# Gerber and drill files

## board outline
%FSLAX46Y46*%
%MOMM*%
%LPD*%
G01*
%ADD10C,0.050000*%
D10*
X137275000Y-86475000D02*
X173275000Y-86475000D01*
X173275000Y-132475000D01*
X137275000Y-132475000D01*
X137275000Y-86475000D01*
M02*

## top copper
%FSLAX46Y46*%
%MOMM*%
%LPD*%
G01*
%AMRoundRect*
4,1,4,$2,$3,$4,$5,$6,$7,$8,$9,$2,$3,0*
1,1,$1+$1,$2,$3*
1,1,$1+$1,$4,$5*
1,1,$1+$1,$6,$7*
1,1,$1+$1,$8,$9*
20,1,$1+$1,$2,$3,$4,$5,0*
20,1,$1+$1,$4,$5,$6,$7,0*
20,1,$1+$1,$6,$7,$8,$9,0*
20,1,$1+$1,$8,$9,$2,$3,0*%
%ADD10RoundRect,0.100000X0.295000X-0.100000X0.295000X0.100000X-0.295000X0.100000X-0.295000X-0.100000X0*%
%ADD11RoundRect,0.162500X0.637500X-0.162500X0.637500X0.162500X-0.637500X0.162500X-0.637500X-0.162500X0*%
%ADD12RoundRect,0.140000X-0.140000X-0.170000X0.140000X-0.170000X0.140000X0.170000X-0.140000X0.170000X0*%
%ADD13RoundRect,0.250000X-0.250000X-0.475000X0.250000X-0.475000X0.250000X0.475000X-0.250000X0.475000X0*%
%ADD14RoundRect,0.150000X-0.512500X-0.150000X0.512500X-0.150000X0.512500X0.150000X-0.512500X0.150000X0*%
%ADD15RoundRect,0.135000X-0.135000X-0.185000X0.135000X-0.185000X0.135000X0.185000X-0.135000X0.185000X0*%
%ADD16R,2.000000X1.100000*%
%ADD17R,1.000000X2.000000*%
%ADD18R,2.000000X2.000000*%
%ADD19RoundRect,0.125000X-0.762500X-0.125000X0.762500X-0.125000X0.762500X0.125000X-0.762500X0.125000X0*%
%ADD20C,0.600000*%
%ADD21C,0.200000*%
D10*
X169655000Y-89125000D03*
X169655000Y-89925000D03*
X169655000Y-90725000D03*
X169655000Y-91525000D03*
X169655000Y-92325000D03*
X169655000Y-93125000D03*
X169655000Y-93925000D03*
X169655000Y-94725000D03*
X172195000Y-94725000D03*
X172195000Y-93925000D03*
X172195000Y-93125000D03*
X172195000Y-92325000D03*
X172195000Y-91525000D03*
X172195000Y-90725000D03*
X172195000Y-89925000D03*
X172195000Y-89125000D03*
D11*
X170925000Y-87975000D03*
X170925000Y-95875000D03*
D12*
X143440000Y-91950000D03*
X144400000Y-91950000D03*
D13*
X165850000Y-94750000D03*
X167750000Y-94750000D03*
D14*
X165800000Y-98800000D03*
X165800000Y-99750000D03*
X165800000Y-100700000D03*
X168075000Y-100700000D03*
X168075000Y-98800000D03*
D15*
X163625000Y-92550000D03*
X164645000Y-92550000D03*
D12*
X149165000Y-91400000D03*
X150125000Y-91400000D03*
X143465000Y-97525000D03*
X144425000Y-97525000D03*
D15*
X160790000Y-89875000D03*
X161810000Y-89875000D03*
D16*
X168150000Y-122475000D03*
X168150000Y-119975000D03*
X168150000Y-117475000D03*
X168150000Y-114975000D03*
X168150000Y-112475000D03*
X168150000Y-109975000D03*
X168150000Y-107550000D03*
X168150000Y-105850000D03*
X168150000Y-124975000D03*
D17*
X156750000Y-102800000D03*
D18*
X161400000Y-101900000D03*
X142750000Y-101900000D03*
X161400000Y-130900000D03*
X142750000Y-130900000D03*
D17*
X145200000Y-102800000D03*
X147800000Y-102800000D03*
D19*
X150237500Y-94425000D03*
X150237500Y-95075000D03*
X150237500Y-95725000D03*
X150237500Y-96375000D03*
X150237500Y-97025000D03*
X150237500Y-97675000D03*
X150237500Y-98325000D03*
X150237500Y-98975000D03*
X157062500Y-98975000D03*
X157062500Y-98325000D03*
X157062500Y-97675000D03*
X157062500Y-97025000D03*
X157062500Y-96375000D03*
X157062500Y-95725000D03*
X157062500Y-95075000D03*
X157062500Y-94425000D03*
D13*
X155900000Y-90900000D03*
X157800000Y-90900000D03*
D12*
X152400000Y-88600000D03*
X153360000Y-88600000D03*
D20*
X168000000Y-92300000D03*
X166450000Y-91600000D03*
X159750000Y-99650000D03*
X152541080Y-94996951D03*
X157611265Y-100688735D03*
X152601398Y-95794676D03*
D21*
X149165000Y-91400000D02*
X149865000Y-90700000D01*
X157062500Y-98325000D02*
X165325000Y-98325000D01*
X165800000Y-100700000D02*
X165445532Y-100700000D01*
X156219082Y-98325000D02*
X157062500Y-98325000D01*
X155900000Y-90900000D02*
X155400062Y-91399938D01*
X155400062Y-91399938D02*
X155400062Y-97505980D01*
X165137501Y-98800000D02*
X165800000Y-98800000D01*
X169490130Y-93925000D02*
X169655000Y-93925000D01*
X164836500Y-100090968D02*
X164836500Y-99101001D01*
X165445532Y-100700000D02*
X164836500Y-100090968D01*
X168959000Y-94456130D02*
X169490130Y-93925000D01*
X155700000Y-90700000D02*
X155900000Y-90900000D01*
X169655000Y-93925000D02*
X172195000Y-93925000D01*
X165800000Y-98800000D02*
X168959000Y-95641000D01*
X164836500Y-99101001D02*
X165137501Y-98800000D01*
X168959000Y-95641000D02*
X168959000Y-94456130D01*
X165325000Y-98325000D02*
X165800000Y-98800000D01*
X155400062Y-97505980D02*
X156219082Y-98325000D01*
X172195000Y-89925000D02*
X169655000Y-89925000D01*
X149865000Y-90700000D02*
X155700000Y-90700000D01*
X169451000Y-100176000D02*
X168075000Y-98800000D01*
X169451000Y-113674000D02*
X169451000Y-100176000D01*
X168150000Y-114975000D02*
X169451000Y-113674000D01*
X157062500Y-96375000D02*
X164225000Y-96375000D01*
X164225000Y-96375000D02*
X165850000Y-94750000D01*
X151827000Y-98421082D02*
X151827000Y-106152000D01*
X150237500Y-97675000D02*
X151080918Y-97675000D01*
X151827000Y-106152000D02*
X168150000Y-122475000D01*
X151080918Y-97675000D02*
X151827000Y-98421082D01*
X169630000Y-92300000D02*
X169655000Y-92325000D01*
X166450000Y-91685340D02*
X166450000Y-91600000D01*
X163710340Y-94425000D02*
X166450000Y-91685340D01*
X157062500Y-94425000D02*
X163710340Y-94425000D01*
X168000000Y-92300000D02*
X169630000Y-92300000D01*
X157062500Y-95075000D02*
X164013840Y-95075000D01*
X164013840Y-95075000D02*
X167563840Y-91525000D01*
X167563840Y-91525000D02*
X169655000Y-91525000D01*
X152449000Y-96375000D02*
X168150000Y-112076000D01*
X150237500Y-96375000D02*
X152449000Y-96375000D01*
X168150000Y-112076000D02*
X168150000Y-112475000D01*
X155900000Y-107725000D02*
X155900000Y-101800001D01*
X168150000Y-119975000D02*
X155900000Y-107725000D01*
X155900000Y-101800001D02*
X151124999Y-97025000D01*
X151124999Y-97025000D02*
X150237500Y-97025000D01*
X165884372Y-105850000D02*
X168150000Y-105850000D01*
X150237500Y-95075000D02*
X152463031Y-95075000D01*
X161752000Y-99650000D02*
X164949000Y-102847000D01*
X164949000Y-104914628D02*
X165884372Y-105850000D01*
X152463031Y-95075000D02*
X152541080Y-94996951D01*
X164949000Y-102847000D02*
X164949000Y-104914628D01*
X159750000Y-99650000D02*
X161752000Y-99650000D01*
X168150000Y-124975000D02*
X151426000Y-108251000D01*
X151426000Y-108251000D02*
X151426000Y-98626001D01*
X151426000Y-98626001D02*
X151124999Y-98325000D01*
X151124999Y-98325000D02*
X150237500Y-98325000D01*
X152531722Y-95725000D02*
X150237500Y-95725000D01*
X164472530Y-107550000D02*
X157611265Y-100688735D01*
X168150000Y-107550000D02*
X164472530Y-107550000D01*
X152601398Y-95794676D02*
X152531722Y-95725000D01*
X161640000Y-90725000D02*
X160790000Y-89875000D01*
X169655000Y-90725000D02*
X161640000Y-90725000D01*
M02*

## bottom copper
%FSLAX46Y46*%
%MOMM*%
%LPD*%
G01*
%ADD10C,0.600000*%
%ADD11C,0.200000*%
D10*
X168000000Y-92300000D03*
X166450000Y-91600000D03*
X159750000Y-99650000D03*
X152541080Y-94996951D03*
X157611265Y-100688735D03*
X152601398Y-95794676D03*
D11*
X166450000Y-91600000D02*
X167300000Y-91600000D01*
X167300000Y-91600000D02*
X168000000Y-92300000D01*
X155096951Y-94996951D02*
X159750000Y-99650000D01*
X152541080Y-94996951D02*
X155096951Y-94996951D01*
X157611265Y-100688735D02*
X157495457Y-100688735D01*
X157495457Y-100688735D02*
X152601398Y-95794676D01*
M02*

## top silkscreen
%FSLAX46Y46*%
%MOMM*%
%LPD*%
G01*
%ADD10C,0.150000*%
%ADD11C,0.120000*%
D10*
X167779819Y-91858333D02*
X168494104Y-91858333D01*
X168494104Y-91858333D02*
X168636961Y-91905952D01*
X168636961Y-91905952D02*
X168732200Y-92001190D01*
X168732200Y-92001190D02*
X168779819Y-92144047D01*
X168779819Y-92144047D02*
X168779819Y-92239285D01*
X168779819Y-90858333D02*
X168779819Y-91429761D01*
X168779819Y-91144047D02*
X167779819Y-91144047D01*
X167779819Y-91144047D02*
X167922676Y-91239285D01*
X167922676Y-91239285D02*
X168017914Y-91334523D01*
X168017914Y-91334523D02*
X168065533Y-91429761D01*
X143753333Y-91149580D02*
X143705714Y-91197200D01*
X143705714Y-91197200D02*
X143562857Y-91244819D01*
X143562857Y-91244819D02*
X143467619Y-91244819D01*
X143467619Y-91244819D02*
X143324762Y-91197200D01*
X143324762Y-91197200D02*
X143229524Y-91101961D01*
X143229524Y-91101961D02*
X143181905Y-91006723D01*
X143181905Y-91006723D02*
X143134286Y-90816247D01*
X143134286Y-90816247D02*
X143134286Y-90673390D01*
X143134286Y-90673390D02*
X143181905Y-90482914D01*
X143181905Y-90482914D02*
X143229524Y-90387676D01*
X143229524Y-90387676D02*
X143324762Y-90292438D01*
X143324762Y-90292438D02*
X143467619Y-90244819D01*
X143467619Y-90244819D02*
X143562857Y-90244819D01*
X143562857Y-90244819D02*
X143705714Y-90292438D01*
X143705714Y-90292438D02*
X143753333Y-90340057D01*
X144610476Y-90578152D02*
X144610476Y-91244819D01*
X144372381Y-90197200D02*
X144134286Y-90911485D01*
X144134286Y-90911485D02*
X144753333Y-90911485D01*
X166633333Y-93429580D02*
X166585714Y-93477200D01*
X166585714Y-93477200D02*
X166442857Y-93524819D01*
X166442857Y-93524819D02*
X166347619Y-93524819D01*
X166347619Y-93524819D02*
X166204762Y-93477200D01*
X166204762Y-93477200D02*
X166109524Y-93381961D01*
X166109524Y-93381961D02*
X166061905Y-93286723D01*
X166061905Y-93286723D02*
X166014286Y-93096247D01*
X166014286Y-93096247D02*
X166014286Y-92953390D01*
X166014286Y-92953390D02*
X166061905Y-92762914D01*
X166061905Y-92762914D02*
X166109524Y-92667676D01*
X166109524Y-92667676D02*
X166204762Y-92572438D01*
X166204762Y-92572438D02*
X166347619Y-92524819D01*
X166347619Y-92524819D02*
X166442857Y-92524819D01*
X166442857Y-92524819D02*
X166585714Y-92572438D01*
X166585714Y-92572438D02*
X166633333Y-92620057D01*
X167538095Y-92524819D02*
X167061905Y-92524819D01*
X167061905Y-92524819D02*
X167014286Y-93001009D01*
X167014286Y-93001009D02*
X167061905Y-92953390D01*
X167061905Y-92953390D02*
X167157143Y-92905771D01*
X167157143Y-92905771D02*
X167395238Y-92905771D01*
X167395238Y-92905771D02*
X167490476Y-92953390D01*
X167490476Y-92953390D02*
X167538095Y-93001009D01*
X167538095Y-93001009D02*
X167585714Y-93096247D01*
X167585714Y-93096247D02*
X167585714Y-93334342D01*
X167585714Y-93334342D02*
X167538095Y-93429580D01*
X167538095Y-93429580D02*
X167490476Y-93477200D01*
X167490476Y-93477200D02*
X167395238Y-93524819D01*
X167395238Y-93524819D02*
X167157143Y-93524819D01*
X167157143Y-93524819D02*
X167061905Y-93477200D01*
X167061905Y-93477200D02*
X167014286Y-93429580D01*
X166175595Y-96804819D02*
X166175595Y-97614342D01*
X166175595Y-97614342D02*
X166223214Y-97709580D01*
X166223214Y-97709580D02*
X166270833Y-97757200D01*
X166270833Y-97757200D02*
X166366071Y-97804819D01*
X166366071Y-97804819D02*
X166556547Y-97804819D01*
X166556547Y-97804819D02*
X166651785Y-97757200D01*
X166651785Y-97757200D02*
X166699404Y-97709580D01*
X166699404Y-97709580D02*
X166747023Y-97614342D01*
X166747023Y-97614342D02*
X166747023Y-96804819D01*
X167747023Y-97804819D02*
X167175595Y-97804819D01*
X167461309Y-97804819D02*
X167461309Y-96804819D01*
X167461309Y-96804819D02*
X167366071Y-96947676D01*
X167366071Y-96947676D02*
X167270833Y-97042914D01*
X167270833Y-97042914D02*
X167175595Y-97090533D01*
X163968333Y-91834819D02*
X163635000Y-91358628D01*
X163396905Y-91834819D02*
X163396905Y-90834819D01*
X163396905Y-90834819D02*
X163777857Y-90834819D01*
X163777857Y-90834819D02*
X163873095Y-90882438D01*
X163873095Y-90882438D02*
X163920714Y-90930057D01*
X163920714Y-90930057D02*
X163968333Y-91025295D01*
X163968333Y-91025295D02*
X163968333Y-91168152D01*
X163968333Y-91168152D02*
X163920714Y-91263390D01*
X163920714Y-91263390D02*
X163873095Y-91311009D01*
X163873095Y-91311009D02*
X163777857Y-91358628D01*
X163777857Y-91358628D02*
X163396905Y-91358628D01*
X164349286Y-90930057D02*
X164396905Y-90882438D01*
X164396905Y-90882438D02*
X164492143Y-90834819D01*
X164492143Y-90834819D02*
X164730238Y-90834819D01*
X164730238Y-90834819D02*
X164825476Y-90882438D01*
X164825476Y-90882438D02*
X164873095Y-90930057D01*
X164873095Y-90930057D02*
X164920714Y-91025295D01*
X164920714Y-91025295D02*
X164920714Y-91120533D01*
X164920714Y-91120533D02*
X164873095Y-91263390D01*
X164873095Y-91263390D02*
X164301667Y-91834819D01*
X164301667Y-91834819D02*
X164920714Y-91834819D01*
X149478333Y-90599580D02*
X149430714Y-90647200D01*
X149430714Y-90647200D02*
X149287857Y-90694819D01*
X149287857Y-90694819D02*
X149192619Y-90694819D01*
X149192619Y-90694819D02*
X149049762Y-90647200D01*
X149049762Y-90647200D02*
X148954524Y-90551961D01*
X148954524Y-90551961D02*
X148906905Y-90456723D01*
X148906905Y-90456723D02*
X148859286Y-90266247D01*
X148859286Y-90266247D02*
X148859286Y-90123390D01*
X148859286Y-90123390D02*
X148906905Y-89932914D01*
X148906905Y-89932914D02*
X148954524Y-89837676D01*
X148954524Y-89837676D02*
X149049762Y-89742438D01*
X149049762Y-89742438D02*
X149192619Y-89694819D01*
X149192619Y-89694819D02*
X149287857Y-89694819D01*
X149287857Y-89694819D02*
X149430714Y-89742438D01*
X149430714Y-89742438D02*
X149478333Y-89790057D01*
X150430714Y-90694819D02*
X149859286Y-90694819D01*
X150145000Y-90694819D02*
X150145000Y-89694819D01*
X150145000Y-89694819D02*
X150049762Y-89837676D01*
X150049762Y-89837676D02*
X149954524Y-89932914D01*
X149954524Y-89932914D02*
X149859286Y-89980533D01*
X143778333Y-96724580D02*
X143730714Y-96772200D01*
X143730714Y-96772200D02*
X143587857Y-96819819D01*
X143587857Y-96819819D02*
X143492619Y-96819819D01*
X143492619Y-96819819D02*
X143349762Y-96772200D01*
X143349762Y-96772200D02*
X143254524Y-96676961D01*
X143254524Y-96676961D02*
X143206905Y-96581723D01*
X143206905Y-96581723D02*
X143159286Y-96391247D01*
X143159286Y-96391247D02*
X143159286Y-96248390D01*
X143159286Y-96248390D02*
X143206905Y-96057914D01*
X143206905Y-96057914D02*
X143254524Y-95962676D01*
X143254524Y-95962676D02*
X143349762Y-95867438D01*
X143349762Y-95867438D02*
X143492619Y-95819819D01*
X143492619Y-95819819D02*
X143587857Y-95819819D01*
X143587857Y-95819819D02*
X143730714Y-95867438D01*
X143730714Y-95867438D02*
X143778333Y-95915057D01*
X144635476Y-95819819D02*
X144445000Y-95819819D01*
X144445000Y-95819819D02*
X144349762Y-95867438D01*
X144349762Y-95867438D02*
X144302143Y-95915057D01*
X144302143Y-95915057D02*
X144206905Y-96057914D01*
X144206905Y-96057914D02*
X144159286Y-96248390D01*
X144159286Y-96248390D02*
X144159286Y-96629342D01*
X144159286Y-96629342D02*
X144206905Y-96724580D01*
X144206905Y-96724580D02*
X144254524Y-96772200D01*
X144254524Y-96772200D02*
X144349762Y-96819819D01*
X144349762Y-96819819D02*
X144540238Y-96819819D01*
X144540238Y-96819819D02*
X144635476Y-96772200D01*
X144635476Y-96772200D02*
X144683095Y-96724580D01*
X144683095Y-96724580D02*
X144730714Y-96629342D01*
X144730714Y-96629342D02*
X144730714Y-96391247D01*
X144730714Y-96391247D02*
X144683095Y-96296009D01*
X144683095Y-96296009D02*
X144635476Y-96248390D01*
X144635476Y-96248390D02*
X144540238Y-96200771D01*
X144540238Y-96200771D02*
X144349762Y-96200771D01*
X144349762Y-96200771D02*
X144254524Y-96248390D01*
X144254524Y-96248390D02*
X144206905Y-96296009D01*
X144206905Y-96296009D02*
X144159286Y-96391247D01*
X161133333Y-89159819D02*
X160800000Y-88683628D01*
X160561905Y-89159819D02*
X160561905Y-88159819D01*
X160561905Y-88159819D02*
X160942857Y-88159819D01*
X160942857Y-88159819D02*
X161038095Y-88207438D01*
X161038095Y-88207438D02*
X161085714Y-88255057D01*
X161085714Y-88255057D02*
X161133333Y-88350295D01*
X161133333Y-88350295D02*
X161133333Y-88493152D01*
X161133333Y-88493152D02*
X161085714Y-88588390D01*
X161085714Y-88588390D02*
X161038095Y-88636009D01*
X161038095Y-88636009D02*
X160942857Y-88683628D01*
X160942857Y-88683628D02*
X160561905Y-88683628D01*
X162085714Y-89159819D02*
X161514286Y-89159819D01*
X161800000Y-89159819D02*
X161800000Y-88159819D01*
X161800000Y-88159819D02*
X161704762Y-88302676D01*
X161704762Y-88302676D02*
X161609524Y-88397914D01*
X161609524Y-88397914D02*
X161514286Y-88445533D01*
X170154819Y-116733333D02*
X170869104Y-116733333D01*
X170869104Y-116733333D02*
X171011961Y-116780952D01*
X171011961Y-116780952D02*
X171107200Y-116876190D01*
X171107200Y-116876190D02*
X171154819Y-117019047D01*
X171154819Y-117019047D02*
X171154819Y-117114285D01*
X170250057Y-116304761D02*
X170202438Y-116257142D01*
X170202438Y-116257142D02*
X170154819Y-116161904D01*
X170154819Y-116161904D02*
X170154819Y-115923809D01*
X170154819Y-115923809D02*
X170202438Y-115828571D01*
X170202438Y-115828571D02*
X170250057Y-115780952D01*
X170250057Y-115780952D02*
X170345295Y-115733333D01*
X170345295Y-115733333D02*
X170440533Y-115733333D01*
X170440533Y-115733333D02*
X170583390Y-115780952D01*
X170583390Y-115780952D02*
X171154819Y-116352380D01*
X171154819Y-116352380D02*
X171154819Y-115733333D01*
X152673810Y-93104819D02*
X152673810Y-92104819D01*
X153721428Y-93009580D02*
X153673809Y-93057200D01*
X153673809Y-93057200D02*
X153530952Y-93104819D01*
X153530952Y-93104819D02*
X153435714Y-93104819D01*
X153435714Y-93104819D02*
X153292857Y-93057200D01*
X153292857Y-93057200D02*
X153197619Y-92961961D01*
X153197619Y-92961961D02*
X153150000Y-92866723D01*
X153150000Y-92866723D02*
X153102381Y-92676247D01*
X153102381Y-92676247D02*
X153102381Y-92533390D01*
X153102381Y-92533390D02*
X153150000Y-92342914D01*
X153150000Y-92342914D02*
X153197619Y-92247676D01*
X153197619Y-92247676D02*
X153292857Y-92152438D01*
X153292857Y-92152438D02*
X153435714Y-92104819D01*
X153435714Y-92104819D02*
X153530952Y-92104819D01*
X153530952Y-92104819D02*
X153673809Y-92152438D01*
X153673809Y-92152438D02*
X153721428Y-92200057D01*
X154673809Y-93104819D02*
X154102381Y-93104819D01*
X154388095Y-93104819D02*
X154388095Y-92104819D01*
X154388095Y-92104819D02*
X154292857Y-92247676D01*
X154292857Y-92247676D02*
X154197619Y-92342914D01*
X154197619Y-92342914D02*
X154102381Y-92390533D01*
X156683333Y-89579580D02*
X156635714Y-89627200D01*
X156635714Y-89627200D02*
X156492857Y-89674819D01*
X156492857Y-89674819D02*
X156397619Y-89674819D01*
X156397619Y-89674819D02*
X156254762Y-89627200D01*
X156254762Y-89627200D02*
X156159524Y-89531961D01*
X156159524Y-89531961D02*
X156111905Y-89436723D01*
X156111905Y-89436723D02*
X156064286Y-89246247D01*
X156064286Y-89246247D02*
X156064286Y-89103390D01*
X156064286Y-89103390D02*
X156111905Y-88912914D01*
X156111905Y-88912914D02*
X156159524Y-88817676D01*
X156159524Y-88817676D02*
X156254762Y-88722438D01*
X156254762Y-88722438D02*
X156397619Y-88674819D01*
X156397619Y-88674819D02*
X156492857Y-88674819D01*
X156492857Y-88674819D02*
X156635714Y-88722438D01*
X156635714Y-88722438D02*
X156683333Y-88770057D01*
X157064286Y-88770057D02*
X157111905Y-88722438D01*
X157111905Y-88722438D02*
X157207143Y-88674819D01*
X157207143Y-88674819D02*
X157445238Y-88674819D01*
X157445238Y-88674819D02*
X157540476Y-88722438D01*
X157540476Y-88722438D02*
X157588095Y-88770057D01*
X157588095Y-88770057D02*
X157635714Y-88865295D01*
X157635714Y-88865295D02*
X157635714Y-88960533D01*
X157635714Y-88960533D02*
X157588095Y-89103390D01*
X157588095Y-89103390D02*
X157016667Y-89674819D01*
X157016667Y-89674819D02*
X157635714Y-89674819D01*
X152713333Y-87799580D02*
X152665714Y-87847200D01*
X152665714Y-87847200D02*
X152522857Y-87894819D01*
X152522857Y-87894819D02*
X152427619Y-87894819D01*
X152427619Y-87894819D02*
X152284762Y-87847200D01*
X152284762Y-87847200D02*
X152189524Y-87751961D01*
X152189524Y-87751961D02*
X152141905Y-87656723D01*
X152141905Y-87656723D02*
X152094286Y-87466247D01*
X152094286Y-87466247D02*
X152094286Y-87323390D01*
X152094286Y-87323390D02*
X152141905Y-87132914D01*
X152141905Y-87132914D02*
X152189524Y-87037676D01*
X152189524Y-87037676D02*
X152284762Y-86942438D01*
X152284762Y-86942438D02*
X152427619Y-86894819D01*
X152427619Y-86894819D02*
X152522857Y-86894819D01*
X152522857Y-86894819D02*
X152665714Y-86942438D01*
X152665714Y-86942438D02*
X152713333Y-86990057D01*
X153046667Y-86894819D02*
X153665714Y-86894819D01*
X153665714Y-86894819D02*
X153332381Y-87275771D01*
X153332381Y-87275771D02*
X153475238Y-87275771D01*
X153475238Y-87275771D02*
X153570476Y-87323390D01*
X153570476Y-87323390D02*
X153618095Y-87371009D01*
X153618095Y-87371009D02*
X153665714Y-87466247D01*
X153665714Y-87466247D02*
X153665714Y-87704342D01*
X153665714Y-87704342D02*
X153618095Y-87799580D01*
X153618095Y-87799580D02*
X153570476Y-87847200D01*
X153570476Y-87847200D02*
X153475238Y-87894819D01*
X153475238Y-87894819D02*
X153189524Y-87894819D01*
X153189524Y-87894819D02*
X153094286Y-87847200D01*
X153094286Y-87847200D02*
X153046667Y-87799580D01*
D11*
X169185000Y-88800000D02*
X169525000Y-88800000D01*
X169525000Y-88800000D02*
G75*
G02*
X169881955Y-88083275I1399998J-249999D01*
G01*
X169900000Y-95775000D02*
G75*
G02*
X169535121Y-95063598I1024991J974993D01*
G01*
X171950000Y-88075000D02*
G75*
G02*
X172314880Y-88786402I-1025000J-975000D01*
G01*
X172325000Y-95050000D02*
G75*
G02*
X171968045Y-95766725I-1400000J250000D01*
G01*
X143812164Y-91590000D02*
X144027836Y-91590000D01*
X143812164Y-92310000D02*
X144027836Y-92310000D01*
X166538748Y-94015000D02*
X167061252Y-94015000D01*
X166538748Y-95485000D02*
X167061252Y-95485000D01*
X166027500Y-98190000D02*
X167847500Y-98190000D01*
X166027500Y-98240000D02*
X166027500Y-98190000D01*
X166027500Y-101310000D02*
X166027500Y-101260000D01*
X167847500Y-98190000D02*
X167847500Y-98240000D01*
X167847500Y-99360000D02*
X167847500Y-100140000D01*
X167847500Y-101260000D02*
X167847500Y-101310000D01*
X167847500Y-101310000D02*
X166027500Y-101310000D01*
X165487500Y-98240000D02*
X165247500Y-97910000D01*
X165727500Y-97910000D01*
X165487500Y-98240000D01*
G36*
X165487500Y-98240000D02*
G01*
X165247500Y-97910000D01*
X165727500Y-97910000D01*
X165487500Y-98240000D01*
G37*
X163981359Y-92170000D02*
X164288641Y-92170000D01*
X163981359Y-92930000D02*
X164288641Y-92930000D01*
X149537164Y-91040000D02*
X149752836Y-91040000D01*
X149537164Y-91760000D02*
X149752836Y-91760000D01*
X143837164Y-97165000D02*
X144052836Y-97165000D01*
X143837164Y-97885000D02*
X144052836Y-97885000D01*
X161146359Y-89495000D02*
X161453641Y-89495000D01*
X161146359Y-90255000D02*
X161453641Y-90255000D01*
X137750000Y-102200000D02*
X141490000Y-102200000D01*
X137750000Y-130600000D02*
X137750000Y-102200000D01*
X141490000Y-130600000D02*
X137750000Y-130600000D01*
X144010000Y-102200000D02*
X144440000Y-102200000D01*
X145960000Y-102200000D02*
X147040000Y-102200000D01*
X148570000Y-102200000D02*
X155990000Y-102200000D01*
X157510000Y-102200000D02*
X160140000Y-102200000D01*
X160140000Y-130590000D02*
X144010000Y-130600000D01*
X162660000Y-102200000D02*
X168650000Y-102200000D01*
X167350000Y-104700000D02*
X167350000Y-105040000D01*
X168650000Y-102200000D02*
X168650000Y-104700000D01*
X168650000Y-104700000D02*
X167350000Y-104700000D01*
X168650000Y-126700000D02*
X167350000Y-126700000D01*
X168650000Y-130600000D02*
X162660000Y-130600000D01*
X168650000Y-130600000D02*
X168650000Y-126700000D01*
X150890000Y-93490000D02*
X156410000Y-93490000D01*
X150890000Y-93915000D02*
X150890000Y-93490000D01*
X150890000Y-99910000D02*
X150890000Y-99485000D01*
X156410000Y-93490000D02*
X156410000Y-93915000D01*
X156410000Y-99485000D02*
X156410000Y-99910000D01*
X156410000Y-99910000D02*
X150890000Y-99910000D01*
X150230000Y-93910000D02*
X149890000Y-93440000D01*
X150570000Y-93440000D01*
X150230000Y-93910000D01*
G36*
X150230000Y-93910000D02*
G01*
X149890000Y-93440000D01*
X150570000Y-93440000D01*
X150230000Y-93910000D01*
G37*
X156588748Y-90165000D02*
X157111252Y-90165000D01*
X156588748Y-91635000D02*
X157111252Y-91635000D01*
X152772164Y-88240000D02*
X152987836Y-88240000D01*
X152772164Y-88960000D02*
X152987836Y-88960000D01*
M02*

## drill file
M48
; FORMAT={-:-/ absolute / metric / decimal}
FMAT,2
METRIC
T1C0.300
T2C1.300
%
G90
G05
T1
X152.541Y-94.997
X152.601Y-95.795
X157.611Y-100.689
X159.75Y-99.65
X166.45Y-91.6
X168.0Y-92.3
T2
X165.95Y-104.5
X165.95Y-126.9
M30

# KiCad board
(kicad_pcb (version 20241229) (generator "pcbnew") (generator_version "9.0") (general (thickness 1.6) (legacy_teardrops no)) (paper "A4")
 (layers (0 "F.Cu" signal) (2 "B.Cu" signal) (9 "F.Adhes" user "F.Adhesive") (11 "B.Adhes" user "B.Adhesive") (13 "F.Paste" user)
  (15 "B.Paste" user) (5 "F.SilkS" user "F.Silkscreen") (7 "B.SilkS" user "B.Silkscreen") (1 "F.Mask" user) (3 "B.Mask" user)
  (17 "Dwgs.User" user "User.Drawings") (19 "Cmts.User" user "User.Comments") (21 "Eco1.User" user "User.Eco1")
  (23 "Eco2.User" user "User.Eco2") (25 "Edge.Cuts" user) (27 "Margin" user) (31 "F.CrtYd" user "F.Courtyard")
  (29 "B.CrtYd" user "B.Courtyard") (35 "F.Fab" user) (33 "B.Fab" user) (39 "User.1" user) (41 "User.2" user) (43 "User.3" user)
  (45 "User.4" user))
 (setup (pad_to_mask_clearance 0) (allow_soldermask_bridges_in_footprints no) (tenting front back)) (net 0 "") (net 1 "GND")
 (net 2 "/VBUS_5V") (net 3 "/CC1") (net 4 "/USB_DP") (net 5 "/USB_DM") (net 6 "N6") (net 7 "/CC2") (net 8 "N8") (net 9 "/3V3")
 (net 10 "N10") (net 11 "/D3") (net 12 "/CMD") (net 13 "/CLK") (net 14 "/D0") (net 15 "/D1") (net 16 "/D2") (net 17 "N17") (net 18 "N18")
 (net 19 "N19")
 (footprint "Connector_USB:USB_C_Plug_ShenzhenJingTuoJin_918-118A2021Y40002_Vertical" (layer "F.Cu") (at 170.925 91.925)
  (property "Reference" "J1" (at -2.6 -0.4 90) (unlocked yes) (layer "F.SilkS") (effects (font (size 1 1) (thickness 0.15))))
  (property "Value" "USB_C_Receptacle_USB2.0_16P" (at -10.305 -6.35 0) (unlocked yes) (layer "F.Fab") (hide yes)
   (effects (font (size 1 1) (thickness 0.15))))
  (fp_line (start -1.74 -3.125) (end -1.4 -3.125) (stroke (width 0.12) (type default)) (layer "F.SilkS"))
  (fp_arc (start -1.4 -3.125) (mid -1.273005 -3.509002) (end -1.043045 -3.841725) (stroke (width 0.12) (type solid)) (layer "F.SilkS"))
  (fp_arc (start -1.025 3.85) (mid -1.258743 3.520613) (end -1.389879 3.138598) (stroke (width 0.12) (type solid)) (layer "F.SilkS"))
  (fp_arc (start 1.025 -3.85) (mid 1.258743 -3.520613) (end 1.389879 -3.138598) (stroke (width 0.12) (type solid)) (layer "F.SilkS"))
  (fp_arc (start 1.4 3.125) (mid 1.273005 3.509002) (end 1.043045 3.841725) (stroke (width 0.12) (type solid)) (layer "F.SilkS"))
  (pad "A1" smd roundrect (at -1.27 -2.8 90) (size 0.4 0.79) (layers "F.Cu" "F.Mask" "F.Paste") (roundrect_rratio 0.25) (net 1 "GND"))
  (pad "A4" smd roundrect (at -1.27 -2 90) (size 0.4 0.79) (layers "F.Cu" "F.Mask" "F.Paste") (roundrect_rratio 0.25) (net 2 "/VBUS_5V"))
  (pad "A5" smd roundrect (at -1.27 -1.2 90) (size 0.4 0.79) (layers "F.Cu" "F.Mask" "F.Paste") (roundrect_rratio 0.25) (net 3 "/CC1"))
  (pad "A6" smd roundrect (at -1.27 -0.4 90) (size 0.4 0.79) (layers "F.Cu" "F.Mask" "F.Paste") (roundrect_rratio 0.25) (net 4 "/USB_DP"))
  (pad "A7" smd roundrect (at -1.27 0.4 90) (size 0.4 0.79) (layers "F.Cu" "F.Mask" "F.Paste") (roundrect_rratio 0.25) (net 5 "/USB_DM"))
  (pad "A8" smd roundrect (at -1.27 1.2 90) (size 0.4 0.79) (layers "F.Cu" "F.Mask" "F.Paste") (roundrect_rratio 0.25) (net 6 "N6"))
  (pad "A9" smd roundrect (at -1.27 2 90) (size 0.4 0.79) (layers "F.Cu" "F.Mask" "F.Paste") (roundrect_rratio 0.25) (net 2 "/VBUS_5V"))
  (pad "A12" smd roundrect (at -1.27 2.8 90) (size 0.4 0.79) (layers "F.Cu" "F.Mask" "F.Paste") (roundrect_rratio 0.25) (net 1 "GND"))
  (pad "B1" smd roundrect (at 1.27 2.8 90) (size 0.4 0.79) (layers "F.Cu" "F.Mask" "F.Paste") (roundrect_rratio 0.25) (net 1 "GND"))
  (pad "B4" smd roundrect (at 1.27 2 90) (size 0.4 0.79) (layers "F.Cu" "F.Mask" "F.Paste") (roundrect_rratio 0.25) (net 2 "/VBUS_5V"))
  (pad "B5" smd roundrect (at 1.27 1.2 90) (size 0.4 0.79) (layers "F.Cu" "F.Mask" "F.Paste") (roundrect_rratio 0.25) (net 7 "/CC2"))
  (pad "B6" smd roundrect (at 1.27 0.4 90) (size 0.4 0.79) (layers "F.Cu" "F.Mask" "F.Paste") (roundrect_rratio 0.25) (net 4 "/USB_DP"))
  (pad "B7" smd roundrect (at 1.27 -0.4 90) (size 0.4 0.79) (layers "F.Cu" "F.Mask" "F.Paste") (roundrect_rratio 0.25) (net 5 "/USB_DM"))
  (pad "B8" smd roundrect (at 1.27 -1.2 90) (size 0.4 0.79) (layers "F.Cu" "F.Mask" "F.Paste") (roundrect_rratio 0.25) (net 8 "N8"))
  (pad "B9" smd roundrect (at 1.27 -2 90) (size 0.4 0.79) (layers "F.Cu" "F.Mask" "F.Paste") (roundrect_rratio 0.25) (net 2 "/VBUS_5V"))
  (pad "B12" smd roundrect (at 1.27 -2.8 90) (size 0.4 0.79) (layers "F.Cu" "F.Mask" "F.Paste") (roundrect_rratio 0.25) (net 1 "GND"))
  (pad "S1" smd roundrect (at 0 -3.95 90) (size 0.65 1.6) (layers "F.Cu" "F.Mask" "F.Paste") (roundrect_rratio 0.25) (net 1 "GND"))
  (pad "S1" smd roundrect (at 0 3.95 90) (size 0.65 1.6) (layers "F.Cu" "F.Mask" "F.Paste") (roundrect_rratio 0.25) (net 1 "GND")))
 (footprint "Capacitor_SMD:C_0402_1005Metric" (layer "F.Cu") (at 143.92 91.95)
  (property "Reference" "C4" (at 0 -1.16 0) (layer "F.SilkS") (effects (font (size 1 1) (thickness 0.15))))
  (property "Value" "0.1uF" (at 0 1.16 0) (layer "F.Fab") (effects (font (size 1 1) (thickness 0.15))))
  (fp_line (start -0.107836 -0.36) (end 0.107836 -0.36) (stroke (width 0.12) (type solid)) (layer "F.SilkS"))
  (fp_line (start -0.107836 0.36) (end 0.107836 0.36) (stroke (width 0.12) (type solid)) (layer "F.SilkS"))
  (pad "1" smd roundrect (at -0.48 0) (size 0.56 0.62) (layers "F.Cu" "F.Mask" "F.Paste") (roundrect_rratio 0.25) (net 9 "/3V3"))
  (pad "2" smd roundrect (at 0.48 0) (size 0.56 0.62) (layers "F.Cu" "F.Mask" "F.Paste") (roundrect_rratio 0.25) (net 1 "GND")))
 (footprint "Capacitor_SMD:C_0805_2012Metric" (layer "F.Cu") (at 166.8 94.75)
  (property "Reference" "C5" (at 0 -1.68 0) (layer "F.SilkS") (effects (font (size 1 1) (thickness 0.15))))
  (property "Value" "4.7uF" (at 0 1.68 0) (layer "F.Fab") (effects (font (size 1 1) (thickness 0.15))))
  (fp_line (start -0.261252 -0.735) (end 0.261252 -0.735) (stroke (width 0.12) (type solid)) (layer "F.SilkS"))
  (fp_line (start -0.261252 0.735) (end 0.261252 0.735) (stroke (width 0.12) (type solid)) (layer "F.SilkS"))
  (pad "1" smd roundrect (at -0.95 0) (size 1 1.45) (layers "F.Cu" "F.Mask" "F.Paste") (roundrect_rratio 0.25) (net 9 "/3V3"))
  (pad "2" smd roundrect (at 0.95 0) (size 1 1.45) (layers "F.Cu" "F.Mask" "F.Paste") (roundrect_rratio 0.25) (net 1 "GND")))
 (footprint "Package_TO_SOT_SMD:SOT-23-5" (layer "F.Cu") (at 166.9375 99.75)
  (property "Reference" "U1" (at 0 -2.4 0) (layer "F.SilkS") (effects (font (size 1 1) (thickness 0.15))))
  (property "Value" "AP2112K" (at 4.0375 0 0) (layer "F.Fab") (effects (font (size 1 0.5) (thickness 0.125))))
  (fp_line (start -0.91 -1.56) (end 0.91 -1.56) (stroke (width 0.12) (type solid)) (layer "F.SilkS"))
  (fp_line (start -0.91 -1.51) (end -0.91 -1.56) (stroke (width 0.12) (type solid)) (layer "F.SilkS"))
  (fp_line (start -0.91 1.56) (end -0.91 1.51) (stroke (width 0.12) (type solid)) (layer "F.SilkS"))
  (fp_line (start 0.91 -1.56) (end 0.91 -1.51) (stroke (width 0.12) (type solid)) (layer "F.SilkS"))
  (fp_line (start 0.91 -0.39) (end 0.91 0.39) (stroke (width 0.12) (type solid)) (layer "F.SilkS"))
  (fp_line (start 0.91 1.51) (end 0.91 1.56) (stroke (width 0.12) (type solid)) (layer "F.SilkS"))
  (fp_line (start 0.91 1.56) (end -0.91 1.56) (stroke (width 0.12) (type solid)) (layer "F.SilkS"))
  (fp_poly (pts (xy -1.45 -1.51) (xy -1.69 -1.84) (xy -1.21 -1.84)) (stroke (width 0.12) (type solid)) (fill yes) (layer "F.SilkS"))
  (pad "1" smd roundrect (at -1.1375 -0.95) (size 1.325 0.6) (layers "F.Cu" "F.Mask" "F.Paste") (roundrect_rratio 0.25) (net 2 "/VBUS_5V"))
  (pad "2" smd roundrect (at -1.1375 0) (size 1.325 0.6) (layers "F.Cu" "F.Mask" "F.Paste") (roundrect_rratio 0.25) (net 1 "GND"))
  (pad "3" smd roundrect (at -1.1375 0.95) (size 1.325 0.6) (layers "F.Cu" "F.Mask" "F.Paste") (roundrect_rratio 0.25) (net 2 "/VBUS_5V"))
  (pad "4" smd roundrect (at 1.1375 0.95) (size 1.325 0.6) (layers "F.Cu" "F.Mask" "F.Paste") (roundrect_rratio 0.25) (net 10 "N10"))
  (pad "5" smd roundrect (at 1.1375 -0.95) (size 1.325 0.6) (layers "F.Cu" "F.Mask" "F.Paste") (roundrect_rratio 0.25) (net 9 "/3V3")))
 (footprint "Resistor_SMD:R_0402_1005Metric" (layer "F.Cu") (at 164.135 92.55)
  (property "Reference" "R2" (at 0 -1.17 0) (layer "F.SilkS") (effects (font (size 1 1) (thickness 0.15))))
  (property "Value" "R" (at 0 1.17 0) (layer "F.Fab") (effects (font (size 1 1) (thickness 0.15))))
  (fp_line (start -0.153641 -0.38) (end 0.153641 -0.38) (stroke (width 0.12) (type solid)) (layer "F.SilkS"))
  (fp_line (start -0.153641 0.38) (end 0.153641 0.38) (stroke (width 0.12) (type solid)) (layer "F.SilkS"))
  (pad "1" smd roundrect (at -0.51 0) (size 0.54 0.64) (layers "F.Cu" "F.Mask" "F.Paste") (roundrect_rratio 0.25) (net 7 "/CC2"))
  (pad "2" smd roundrect (at 0.51 0) (size 0.54 0.64) (layers "F.Cu" "F.Mask" "F.Paste") (roundrect_rratio 0.25) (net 1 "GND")))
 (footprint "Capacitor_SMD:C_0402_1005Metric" (layer "F.Cu") (at 149.645 91.4)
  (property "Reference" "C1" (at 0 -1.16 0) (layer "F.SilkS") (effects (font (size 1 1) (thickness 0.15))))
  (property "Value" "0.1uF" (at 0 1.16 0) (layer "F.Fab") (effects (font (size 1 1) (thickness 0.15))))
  (fp_line (start -0.107836 -0.36) (end 0.107836 -0.36) (stroke (width 0.12) (type solid)) (layer "F.SilkS"))
  (fp_line (start -0.107836 0.36) (end 0.107836 0.36) (stroke (width 0.12) (type solid)) (layer "F.SilkS"))
  (pad "1" smd roundrect (at -0.48 0) (size 0.56 0.62) (layers "F.Cu" "F.Mask" "F.Paste") (roundrect_rratio 0.25) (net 2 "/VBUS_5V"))
  (pad "2" smd roundrect (at 0.48 0) (size 0.56 0.62) (layers "F.Cu" "F.Mask" "F.Paste") (roundrect_rratio 0.25) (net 1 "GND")))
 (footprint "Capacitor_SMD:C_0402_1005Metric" (layer "F.Cu") (at 143.945 97.525)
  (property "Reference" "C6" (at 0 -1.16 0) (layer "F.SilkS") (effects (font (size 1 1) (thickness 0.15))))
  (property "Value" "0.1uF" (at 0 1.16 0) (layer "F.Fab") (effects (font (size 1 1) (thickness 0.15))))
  (fp_line (start -0.107836 -0.36) (end 0.107836 -0.36) (stroke (width 0.12) (type solid)) (layer "F.SilkS"))
  (fp_line (start -0.107836 0.36) (end 0.107836 0.36) (stroke (width 0.12) (type solid)) (layer "F.SilkS"))
  (pad "1" smd roundrect (at -0.48 0) (size 0.56 0.62) (layers "F.Cu" "F.Mask" "F.Paste") (roundrect_rratio 0.25) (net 9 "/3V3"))
  (pad "2" smd roundrect (at 0.48 0) (size 0.56 0.62) (layers "F.Cu" "F.Mask" "F.Paste") (roundrect_rratio 0.25) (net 1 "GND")))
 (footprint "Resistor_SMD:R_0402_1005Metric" (layer "F.Cu") (at 161.3 89.875)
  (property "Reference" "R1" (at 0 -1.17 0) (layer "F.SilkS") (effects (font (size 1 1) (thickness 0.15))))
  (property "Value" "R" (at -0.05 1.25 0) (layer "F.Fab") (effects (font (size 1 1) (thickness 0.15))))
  (fp_line (start -0.153641 -0.38) (end 0.153641 -0.38) (stroke (width 0.12) (type solid)) (layer "F.SilkS"))
  (fp_line (start -0.153641 0.38) (end 0.153641 0.38) (stroke (width 0.12) (type solid)) (layer "F.SilkS"))
  (pad "1" smd roundrect (at -0.51 0) (size 0.54 0.64) (layers "F.Cu" "F.Mask" "F.Paste") (roundrect_rratio 0.25) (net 3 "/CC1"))
  (pad "2" smd roundrect (at 0.51 0) (size 0.54 0.64) (layers "F.Cu" "F.Mask" "F.Paste") (roundrect_rratio 0.25) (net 1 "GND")))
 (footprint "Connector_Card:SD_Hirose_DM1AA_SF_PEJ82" (layer "F.Cu") (at 153.2 116.4 -90)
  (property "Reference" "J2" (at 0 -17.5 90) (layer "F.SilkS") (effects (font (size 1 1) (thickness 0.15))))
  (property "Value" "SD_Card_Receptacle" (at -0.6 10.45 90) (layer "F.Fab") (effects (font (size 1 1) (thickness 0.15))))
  (fp_line (start -14.2 15.45) (end -14.2 11.71) (stroke (width 0.12) (type solid)) (layer "F.SilkS"))
  (fp_line (start 14.2 15.45) (end -14.2 15.45) (stroke (width 0.12) (type solid)) (layer "F.SilkS"))
  (fp_line (start 14.2 11.71) (end 14.2 15.45) (stroke (width 0.12) (type solid)) (layer "F.SilkS"))
  (fp_line (start -14.2 9.19) (end -14.2 8.76) (stroke (width 0.12) (type solid)) (layer "F.SilkS"))
  (fp_line (start -14.2 7.24) (end -14.2 6.16) (stroke (width 0.12) (type solid)) (layer "F.SilkS"))
  (fp_line (start -14.2 4.63) (end -14.2 -2.79) (stroke (width 0.12) (type solid)) (layer "F.SilkS"))
  (fp_line (start -14.2 -4.31) (end -14.2 -6.94) (stroke (width 0.12) (type solid)) (layer "F.SilkS"))
  (fp_line (start 14.19 -6.94) (end 14.2 9.19) (stroke (width 0.12) (type solid)) (layer "F.SilkS"))
  (fp_line (start -14.2 -9.46) (end -14.2 -15.45) (stroke (width 0.12) (type solid)) (layer "F.SilkS"))
  (fp_line (start -11.7 -14.15) (end -11.36 -14.15) (stroke (width 0.12) (type solid)) (layer "F.SilkS"))
  (fp_line (start -14.2 -15.45) (end -11.7 -15.45) (stroke (width 0.12) (type solid)) (layer "F.SilkS"))
  (fp_line (start -11.7 -15.45) (end -11.7 -14.15) (stroke (width 0.12) (type solid)) (layer "F.SilkS"))
  (fp_line (start 10.3 -15.45) (end 10.3 -14.15) (stroke (width 0.12) (type solid)) (layer "F.SilkS"))
  (fp_line (start 14.2 -15.45) (end 14.2 -9.46) (stroke (width 0.12) (type solid)) (layer "F.SilkS"))
  (fp_line (start 14.2 -15.45) (end 10.3 -15.45) (stroke (width 0.12) (type solid)) (layer "F.SilkS"))
  (pad "" np_thru_hole circle (at -11.9 -12.75 270) (size 1.3 1.3) (drill 1.3) (layers "*.Cu" "*.Mask"))
  (pad "" np_thru_hole circle (at 10.5 -12.75 270) (size 1.3 1.3) (drill 1.3) (layers "*.Cu" "*.Mask"))
  (pad "1" smd rect (at 6.075 -14.95 270) (size 1.1 2) (layers "F.Cu" "F.Mask" "F.Paste") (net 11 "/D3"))
  (pad "2" smd rect (at 3.575 -14.95 270) (size 1.1 2) (layers "F.Cu" "F.Mask" "F.Paste") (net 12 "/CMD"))
  (pad "3" smd rect (at 1.075 -14.95 270) (size 1.1 2) (layers "F.Cu" "F.Mask" "F.Paste") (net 1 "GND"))
  (pad "4" smd rect (at -1.425 -14.95 270) (size 1.1 2) (layers "F.Cu" "F.Mask" "F.Paste") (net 9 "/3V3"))
  (pad "5" smd rect (at -3.925 -14.95 270) (size 1.1 2) (layers "F.Cu" "F.Mask" "F.Paste") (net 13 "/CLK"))
  (pad "6" smd rect (at -6.425 -14.95 270) (size 1.1 2) (layers "F.Cu" "F.Mask" "F.Paste") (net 1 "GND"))
  (pad "7" smd rect (at -8.85 -14.95 270) (size 1.1 2) (layers "F.Cu" "F.Mask" "F.Paste") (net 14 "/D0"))
  (pad "8" smd rect (at -10.55 -14.95 270) (size 1.1 2) (layers "F.Cu" "F.Mask" "F.Paste") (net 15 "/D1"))
  (pad "9" smd rect (at 8.575 -14.95 270) (size 1.1 2) (layers "F.Cu" "F.Mask" "F.Paste") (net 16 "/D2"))
  (pad "CP" smd rect (at -13.6 -3.55 270) (size 2 1) (layers "F.Cu" "F.Mask" "F.Paste"))
  (pad "SH" smd rect (at -14.5 -8.2 270) (size 2 2) (layers "F.Cu" "F.Mask" "F.Paste"))
  (pad "SH" smd rect (at -14.5 10.45 270) (size 2 2) (layers "F.Cu" "F.Mask" "F.Paste"))
  (pad "SH" smd rect (at 14.5 -8.2 270) (size 2 2) (layers "F.Cu" "F.Mask" "F.Paste"))
  (pad "SH" smd rect (at 14.5 10.45 270) (size 2 2) (layers "F.Cu" "F.Mask" "F.Paste"))
  (pad "SW" smd rect (at -13.6 8 270) (size 2 1) (layers "F.Cu" "F.Mask" "F.Paste"))
  (pad "WP" smd rect (at -13.6 5.4 270) (size 2 1) (layers "F.Cu" "F.Mask" "F.Paste")))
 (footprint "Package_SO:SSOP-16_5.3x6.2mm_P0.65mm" (layer "F.Cu") (at 153.65 96.7)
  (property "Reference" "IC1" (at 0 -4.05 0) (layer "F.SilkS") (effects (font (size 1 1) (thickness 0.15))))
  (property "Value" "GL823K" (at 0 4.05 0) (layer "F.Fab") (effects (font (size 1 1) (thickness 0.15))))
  (fp_line (start -2.76 -3.21) (end 2.76 -3.21) (stroke (width 0.12) (type solid)) (layer "F.SilkS"))
  (fp_line (start -2.76 -2.785) (end -2.76 -3.21) (stroke (width 0.12) (type solid)) (layer "F.SilkS"))
  (fp_line (start -2.76 3.21) (end -2.76 2.785) (stroke (width 0.12) (type solid)) (layer "F.SilkS"))
  (fp_line (start 2.76 -3.21) (end 2.76 -2.785) (stroke (width 0.12) (type solid)) (layer "F.SilkS"))
  (fp_line (start 2.76 2.785) (end 2.76 3.21) (stroke (width 0.12) (type solid)) (layer "F.SilkS"))
  (fp_line (start 2.76 3.21) (end -2.76 3.21) (stroke (width 0.12) (type solid)) (layer "F.SilkS"))
  (fp_poly (pts (xy -3.42 -2.79) (xy -3.76 -3.26) (xy -3.08 -3.26)) (stroke (width 0.12) (type solid)) (fill yes) (layer "F.SilkS"))
  (pad "1" smd roundrect (at -3.4125 -2.275) (size 1.775 0.5) (layers "F.Cu" "F.Mask" "F.Paste") (roundrect_rratio 0.25) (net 1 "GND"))
  (pad "2" smd roundrect (at -3.4125 -1.625) (size 1.775 0.5) (layers "F.Cu" "F.Mask" "F.Paste") (roundrect_rratio 0.25) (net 15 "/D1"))
  (pad "3" smd roundrect (at -3.4125 -0.975) (size 1.775 0.5) (layers "F.Cu" "F.Mask" "F.Paste") (roundrect_rratio 0.25) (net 14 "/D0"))
  (pad "4" smd roundrect (at -3.4125 -0.325) (size 1.775 0.5) (layers "F.Cu" "F.Mask" "F.Paste") (roundrect_rratio 0.25) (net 13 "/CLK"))
  (pad "5" smd roundrect (at -3.4125 0.325) (size 1.775 0.5) (layers "F.Cu" "F.Mask" "F.Paste") (roundrect_rratio 0.25) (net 12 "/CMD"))
  (pad "6" smd roundrect (at -3.4125 0.975) (size 1.775 0.5) (layers "F.Cu" "F.Mask" "F.Paste") (roundrect_rratio 0.25) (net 11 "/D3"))
  (pad "7" smd roundrect (at -3.4125 1.625) (size 1.775 0.5) (layers "F.Cu" "F.Mask" "F.Paste") (roundrect_rratio 0.25) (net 16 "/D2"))
  (pad "8" smd roundrect (at -3.4125 2.275) (size 1.775 0.5) (layers "F.Cu" "F.Mask" "F.Paste") (roundrect_rratio 0.25) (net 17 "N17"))
  (pad "9" smd roundrect (at 3.4125 2.275) (size 1.775 0.5) (layers "F.Cu" "F.Mask" "F.Paste") (roundrect_rratio 0.25) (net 9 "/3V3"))
  (pad "10" smd roundrect (at 3.4125 1.625) (size 1.775 0.5) (layers "F.Cu" "F.Mask" "F.Paste") (roundrect_rratio 0.25) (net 2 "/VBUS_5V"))
  (pad "11" smd roundrect (at 3.4125 0.975) (size 1.775 0.5) (layers "F.Cu" "F.Mask" "F.Paste") (roundrect_rratio 0.25) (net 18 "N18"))
  (pad "12" smd roundrect (at 3.4125 0.325) (size 1.775 0.5) (layers "F.Cu" "F.Mask" "F.Paste") (roundrect_rratio 0.25) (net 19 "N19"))
  (pad "13" smd roundrect (at 3.4125 -0.325) (size 1.775 0.5) (layers "F.Cu" "F.Mask" "F.Paste") (roundrect_rratio 0.25) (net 9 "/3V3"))
  (pad "14" smd roundrect (at 3.4125 -0.975) (size 1.775 0.5) (layers "F.Cu" "F.Mask" "F.Paste") (roundrect_rratio 0.25) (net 1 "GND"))
  (pad "15" smd roundrect (at 3.4125 -1.625) (size 1.775 0.5) (layers "F.Cu" "F.Mask" "F.Paste") (roundrect_rratio 0.25) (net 4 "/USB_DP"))
  (pad "16" smd roundrect (at 3.4125 -2.275) (size 1.775 0.5) (layers "F.Cu" "F.Mask" "F.Paste") (roundrect_rratio 0.25) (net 5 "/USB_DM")))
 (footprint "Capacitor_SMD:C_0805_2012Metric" (layer "F.Cu") (at 156.85 90.9)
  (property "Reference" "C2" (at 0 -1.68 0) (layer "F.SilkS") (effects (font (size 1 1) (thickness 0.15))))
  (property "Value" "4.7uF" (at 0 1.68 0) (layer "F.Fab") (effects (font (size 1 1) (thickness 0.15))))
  (fp_line (start -0.261252 -0.735) (end 0.261252 -0.735) (stroke (width 0.12) (type solid)) (layer "F.SilkS"))
  (fp_line (start -0.261252 0.735) (end 0.261252 0.735) (stroke (width 0.12) (type solid)) (layer "F.SilkS"))
  (pad "1" smd roundrect (at -0.95 0) (size 1 1.45) (layers "F.Cu" "F.Mask" "F.Paste") (roundrect_rratio 0.25) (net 2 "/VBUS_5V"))
  (pad "2" smd roundrect (at 0.95 0) (size 1 1.45) (layers "F.Cu" "F.Mask" "F.Paste") (roundrect_rratio 0.25) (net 1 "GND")))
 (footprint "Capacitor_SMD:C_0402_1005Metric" (layer "F.Cu") (at 152.88 88.6)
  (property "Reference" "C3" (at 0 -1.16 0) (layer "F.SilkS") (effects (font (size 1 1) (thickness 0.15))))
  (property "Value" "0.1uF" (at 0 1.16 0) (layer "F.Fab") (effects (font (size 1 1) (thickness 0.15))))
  (fp_line (start -0.107836 -0.36) (end 0.107836 -0.36) (stroke (width 0.12) (type solid)) (layer "F.SilkS"))
  (fp_line (start -0.107836 0.36) (end 0.107836 0.36) (stroke (width 0.12) (type solid)) (layer "F.SilkS"))
  (pad "1" smd roundrect (at -0.48 0) (size 0.56 0.62) (layers "F.Cu" "F.Mask" "F.Paste") (roundrect_rratio 0.25) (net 9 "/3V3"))
  (pad "2" smd roundrect (at 0.48 0) (size 0.56 0.62) (layers "F.Cu" "F.Mask" "F.Paste") (roundrect_rratio 0.25) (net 1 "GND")))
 (gr_rect (start 137.275 86.475) (end 173.275 132.475) (stroke (width 0.05) (type solid)) (fill no) (layer "Edge.Cuts"))
 (segment (start 149.165 91.4) (end 149.865 90.7) (width 0.2) (layer "F.Cu") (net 2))
 (segment (start 157.0625 98.325) (end 165.325 98.325) (width 0.2) (layer "F.Cu") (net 2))
 (segment (start 165.8 100.7) (end 165.445532 100.7) (width 0.2) (layer "F.Cu") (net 2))
 (segment (start 156.219082 98.325) (end 157.0625 98.325) (width 0.2) (layer "F.Cu") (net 2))
 (segment (start 155.9 90.9) (end 155.400062 91.399938) (width 0.2) (layer "F.Cu") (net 2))
 (segment (start 155.400062 91.399938) (end 155.400062 97.50598) (width 0.2) (layer "F.Cu") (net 2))
 (segment (start 165.137501 98.8) (end 165.8 98.8) (width 0.2) (layer "F.Cu") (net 2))
 (segment (start 169.49013 93.925) (end 169.655 93.925) (width 0.2) (layer "F.Cu") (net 2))
 (segment (start 164.8365 100.090968) (end 164.8365 99.101001) (width 0.2) (layer "F.Cu") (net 2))
 (segment (start 165.445532 100.7) (end 164.8365 100.090968) (width 0.2) (layer "F.Cu") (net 2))
 (segment (start 168.959 94.45613) (end 169.49013 93.925) (width 0.2) (layer "F.Cu") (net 2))
 (segment (start 155.7 90.7) (end 155.9 90.9) (width 0.2) (layer "F.Cu") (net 2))
 (segment (start 169.655 93.925) (end 172.195 93.925) (width 0.2) (layer "F.Cu") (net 2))
 (segment (start 165.8 98.8) (end 168.959 95.641) (width 0.2) (layer "F.Cu") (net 2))
 (segment (start 164.8365 99.101001) (end 165.137501 98.8) (width 0.2) (layer "F.Cu") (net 2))
 (segment (start 168.959 95.641) (end 168.959 94.45613) (width 0.2) (layer "F.Cu") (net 2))
 (segment (start 165.325 98.325) (end 165.8 98.8) (width 0.2) (layer "F.Cu") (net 2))
 (segment (start 155.400062 97.50598) (end 156.219082 98.325) (width 0.2) (layer "F.Cu") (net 2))
 (segment (start 172.195 89.925) (end 169.655 89.925) (width 0.2) (layer "F.Cu") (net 2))
 (segment (start 149.865 90.7) (end 155.7 90.7) (width 0.2) (layer "F.Cu") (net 2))
 (segment (start 169.451 100.176) (end 168.075 98.8) (width 0.2) (layer "F.Cu") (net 9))
 (segment (start 169.451 113.674) (end 169.451 100.176) (width 0.2) (layer "F.Cu") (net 9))
 (segment (start 168.15 114.975) (end 169.451 113.674) (width 0.2) (layer "F.Cu") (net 9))
 (segment (start 157.0625 96.375) (end 164.225 96.375) (width 0.2) (layer "F.Cu") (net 9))
 (segment (start 164.225 96.375) (end 165.85 94.75) (width 0.2) (layer "F.Cu") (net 9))
 (segment (start 151.827 98.421082) (end 151.827 106.152) (width 0.2) (layer "F.Cu") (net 11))
 (segment (start 150.2375 97.675) (end 151.080918 97.675) (width 0.2) (layer "F.Cu") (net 11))
 (segment (start 151.827 106.152) (end 168.15 122.475) (width 0.2) (layer "F.Cu") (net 11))
 (segment (start 151.080918 97.675) (end 151.827 98.421082) (width 0.2) (layer "F.Cu") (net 11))
 (segment (start 169.63 92.3) (end 169.655 92.325) (width 0.2) (layer "F.Cu") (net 5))
 (segment (start 166.45 91.68534) (end 166.45 91.6) (width 0.2) (layer "F.Cu") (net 5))
 (segment (start 163.71034 94.425) (end 166.45 91.68534) (width 0.2) (layer "F.Cu") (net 5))
 (segment (start 157.0625 94.425) (end 163.71034 94.425) (width 0.2) (layer "F.Cu") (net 5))
 (segment (start 168 92.3) (end 169.63 92.3) (width 0.2) (layer "F.Cu") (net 5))
 (via (at 168 92.3) (size 0.6) (drill 0.3) (layers "F.Cu" "B.Cu") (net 5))
 (via (at 166.45 91.6) (size 0.6) (drill 0.3) (layers "F.Cu" "B.Cu") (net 5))
 (segment (start 166.45 91.6) (end 167.3 91.6) (width 0.2) (layer "B.Cu") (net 5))
 (segment (start 167.3 91.6) (end 168 92.3) (width 0.2) (layer "B.Cu") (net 5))
 (segment (start 157.0625 95.075) (end 164.01384 95.075) (width 0.2) (layer "F.Cu") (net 4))
 (segment (start 164.01384 95.075) (end 167.56384 91.525) (width 0.2) (layer "F.Cu") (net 4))
 (segment (start 167.56384 91.525) (end 169.655 91.525) (width 0.2) (layer "F.Cu") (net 4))
 (segment (start 152.449 96.375) (end 168.15 112.076) (width 0.2) (layer "F.Cu") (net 13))
 (segment (start 150.2375 96.375) (end 152.449 96.375) (width 0.2) (layer "F.Cu") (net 13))
 (segment (start 168.15 112.076) (end 168.15 112.475) (width 0.2) (layer "F.Cu") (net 13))
 (segment (start 155.9 107.725) (end 155.9 101.800001) (width 0.2) (layer "F.Cu") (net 12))
 (segment (start 168.15 119.975) (end 155.9 107.725) (width 0.2) (layer "F.Cu") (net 12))
 (segment (start 155.9 101.800001) (end 151.124999 97.025) (width 0.2) (layer "F.Cu") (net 12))
 (segment (start 151.124999 97.025) (end 150.2375 97.025) (width 0.2) (layer "F.Cu") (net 12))
 (segment (start 165.884372 105.85) (end 168.15 105.85) (width 0.2) (layer "F.Cu") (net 15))
 (segment (start 150.2375 95.075) (end 152.463031 95.075) (width 0.2) (layer "F.Cu") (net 15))
 (segment (start 161.752 99.65) (end 164.949 102.847) (width 0.2) (layer "F.Cu") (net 15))
 (segment (start 164.949 104.914628) (end 165.884372 105.85) (width 0.2) (layer "F.Cu") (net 15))
 (segment (start 152.463031 95.075) (end 152.54108 94.996951) (width 0.2) (layer "F.Cu") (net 15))
 (segment (start 164.949 102.847) (end 164.949 104.914628) (width 0.2) (layer "F.Cu") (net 15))
 (segment (start 159.75 99.65) (end 161.752 99.65) (width 0.2) (layer "F.Cu") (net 15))
 (via (at 159.75 99.65) (size 0.6) (drill 0.3) (layers "F.Cu" "B.Cu") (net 15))
 (via (at 152.54108 94.996951) (size 0.6) (drill 0.3) (layers "F.Cu" "B.Cu") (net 15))
 (segment (start 155.096951 94.996951) (end 159.75 99.65) (width 0.2) (layer "B.Cu") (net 15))
 (segment (start 152.54108 94.996951) (end 155.096951 94.996951) (width 0.2) (layer "B.Cu") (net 15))
 (segment (start 168.15 124.975) (end 151.426 108.251) (width 0.2) (layer "F.Cu") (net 16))
 (segment (start 151.426 108.251) (end 151.426 98.626001) (width 0.2) (layer "F.Cu") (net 16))
 (segment (start 151.426 98.626001) (end 151.124999 98.325) (width 0.2) (layer "F.Cu") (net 16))
 (segment (start 151.124999 98.325) (end 150.2375 98.325) (width 0.2) (layer "F.Cu") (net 16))
 (segment (start 152.531722 95.725) (end 150.2375 95.725) (width 0.2) (layer "F.Cu") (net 14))
 (segment (start 164.47253 107.55) (end 157.611265 100.688735) (width 0.2) (layer "F.Cu") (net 14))
 (segment (start 168.15 107.55) (end 164.47253 107.55) (width 0.2) (layer "F.Cu") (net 14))
 (segment (start 152.601398 95.794676) (end 152.531722 95.725) (width 0.2) (layer "F.Cu") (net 14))
 (via (at 157.611265 100.688735) (size 0.6) (drill 0.3) (layers "F.Cu" "B.Cu") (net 14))
 (via (at 152.601398 95.794676) (size 0.6) (drill 0.3) (layers "F.Cu" "B.Cu") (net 14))
 (segment (start 157.611265 100.688735) (end 157.495457 100.688735) (width 0.2) (layer "B.Cu") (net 14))
 (segment (start 157.495457 100.688735) (end 152.601398 95.794676) (width 0.2) (layer "B.Cu") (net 14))
 (segment (start 161.64 90.725) (end 160.79 89.875) (width 0.2) (layer "F.Cu") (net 3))
 (segment (start 169.655 90.725) (end 161.64 90.725) (width 0.2) (layer "F.Cu") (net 3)))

